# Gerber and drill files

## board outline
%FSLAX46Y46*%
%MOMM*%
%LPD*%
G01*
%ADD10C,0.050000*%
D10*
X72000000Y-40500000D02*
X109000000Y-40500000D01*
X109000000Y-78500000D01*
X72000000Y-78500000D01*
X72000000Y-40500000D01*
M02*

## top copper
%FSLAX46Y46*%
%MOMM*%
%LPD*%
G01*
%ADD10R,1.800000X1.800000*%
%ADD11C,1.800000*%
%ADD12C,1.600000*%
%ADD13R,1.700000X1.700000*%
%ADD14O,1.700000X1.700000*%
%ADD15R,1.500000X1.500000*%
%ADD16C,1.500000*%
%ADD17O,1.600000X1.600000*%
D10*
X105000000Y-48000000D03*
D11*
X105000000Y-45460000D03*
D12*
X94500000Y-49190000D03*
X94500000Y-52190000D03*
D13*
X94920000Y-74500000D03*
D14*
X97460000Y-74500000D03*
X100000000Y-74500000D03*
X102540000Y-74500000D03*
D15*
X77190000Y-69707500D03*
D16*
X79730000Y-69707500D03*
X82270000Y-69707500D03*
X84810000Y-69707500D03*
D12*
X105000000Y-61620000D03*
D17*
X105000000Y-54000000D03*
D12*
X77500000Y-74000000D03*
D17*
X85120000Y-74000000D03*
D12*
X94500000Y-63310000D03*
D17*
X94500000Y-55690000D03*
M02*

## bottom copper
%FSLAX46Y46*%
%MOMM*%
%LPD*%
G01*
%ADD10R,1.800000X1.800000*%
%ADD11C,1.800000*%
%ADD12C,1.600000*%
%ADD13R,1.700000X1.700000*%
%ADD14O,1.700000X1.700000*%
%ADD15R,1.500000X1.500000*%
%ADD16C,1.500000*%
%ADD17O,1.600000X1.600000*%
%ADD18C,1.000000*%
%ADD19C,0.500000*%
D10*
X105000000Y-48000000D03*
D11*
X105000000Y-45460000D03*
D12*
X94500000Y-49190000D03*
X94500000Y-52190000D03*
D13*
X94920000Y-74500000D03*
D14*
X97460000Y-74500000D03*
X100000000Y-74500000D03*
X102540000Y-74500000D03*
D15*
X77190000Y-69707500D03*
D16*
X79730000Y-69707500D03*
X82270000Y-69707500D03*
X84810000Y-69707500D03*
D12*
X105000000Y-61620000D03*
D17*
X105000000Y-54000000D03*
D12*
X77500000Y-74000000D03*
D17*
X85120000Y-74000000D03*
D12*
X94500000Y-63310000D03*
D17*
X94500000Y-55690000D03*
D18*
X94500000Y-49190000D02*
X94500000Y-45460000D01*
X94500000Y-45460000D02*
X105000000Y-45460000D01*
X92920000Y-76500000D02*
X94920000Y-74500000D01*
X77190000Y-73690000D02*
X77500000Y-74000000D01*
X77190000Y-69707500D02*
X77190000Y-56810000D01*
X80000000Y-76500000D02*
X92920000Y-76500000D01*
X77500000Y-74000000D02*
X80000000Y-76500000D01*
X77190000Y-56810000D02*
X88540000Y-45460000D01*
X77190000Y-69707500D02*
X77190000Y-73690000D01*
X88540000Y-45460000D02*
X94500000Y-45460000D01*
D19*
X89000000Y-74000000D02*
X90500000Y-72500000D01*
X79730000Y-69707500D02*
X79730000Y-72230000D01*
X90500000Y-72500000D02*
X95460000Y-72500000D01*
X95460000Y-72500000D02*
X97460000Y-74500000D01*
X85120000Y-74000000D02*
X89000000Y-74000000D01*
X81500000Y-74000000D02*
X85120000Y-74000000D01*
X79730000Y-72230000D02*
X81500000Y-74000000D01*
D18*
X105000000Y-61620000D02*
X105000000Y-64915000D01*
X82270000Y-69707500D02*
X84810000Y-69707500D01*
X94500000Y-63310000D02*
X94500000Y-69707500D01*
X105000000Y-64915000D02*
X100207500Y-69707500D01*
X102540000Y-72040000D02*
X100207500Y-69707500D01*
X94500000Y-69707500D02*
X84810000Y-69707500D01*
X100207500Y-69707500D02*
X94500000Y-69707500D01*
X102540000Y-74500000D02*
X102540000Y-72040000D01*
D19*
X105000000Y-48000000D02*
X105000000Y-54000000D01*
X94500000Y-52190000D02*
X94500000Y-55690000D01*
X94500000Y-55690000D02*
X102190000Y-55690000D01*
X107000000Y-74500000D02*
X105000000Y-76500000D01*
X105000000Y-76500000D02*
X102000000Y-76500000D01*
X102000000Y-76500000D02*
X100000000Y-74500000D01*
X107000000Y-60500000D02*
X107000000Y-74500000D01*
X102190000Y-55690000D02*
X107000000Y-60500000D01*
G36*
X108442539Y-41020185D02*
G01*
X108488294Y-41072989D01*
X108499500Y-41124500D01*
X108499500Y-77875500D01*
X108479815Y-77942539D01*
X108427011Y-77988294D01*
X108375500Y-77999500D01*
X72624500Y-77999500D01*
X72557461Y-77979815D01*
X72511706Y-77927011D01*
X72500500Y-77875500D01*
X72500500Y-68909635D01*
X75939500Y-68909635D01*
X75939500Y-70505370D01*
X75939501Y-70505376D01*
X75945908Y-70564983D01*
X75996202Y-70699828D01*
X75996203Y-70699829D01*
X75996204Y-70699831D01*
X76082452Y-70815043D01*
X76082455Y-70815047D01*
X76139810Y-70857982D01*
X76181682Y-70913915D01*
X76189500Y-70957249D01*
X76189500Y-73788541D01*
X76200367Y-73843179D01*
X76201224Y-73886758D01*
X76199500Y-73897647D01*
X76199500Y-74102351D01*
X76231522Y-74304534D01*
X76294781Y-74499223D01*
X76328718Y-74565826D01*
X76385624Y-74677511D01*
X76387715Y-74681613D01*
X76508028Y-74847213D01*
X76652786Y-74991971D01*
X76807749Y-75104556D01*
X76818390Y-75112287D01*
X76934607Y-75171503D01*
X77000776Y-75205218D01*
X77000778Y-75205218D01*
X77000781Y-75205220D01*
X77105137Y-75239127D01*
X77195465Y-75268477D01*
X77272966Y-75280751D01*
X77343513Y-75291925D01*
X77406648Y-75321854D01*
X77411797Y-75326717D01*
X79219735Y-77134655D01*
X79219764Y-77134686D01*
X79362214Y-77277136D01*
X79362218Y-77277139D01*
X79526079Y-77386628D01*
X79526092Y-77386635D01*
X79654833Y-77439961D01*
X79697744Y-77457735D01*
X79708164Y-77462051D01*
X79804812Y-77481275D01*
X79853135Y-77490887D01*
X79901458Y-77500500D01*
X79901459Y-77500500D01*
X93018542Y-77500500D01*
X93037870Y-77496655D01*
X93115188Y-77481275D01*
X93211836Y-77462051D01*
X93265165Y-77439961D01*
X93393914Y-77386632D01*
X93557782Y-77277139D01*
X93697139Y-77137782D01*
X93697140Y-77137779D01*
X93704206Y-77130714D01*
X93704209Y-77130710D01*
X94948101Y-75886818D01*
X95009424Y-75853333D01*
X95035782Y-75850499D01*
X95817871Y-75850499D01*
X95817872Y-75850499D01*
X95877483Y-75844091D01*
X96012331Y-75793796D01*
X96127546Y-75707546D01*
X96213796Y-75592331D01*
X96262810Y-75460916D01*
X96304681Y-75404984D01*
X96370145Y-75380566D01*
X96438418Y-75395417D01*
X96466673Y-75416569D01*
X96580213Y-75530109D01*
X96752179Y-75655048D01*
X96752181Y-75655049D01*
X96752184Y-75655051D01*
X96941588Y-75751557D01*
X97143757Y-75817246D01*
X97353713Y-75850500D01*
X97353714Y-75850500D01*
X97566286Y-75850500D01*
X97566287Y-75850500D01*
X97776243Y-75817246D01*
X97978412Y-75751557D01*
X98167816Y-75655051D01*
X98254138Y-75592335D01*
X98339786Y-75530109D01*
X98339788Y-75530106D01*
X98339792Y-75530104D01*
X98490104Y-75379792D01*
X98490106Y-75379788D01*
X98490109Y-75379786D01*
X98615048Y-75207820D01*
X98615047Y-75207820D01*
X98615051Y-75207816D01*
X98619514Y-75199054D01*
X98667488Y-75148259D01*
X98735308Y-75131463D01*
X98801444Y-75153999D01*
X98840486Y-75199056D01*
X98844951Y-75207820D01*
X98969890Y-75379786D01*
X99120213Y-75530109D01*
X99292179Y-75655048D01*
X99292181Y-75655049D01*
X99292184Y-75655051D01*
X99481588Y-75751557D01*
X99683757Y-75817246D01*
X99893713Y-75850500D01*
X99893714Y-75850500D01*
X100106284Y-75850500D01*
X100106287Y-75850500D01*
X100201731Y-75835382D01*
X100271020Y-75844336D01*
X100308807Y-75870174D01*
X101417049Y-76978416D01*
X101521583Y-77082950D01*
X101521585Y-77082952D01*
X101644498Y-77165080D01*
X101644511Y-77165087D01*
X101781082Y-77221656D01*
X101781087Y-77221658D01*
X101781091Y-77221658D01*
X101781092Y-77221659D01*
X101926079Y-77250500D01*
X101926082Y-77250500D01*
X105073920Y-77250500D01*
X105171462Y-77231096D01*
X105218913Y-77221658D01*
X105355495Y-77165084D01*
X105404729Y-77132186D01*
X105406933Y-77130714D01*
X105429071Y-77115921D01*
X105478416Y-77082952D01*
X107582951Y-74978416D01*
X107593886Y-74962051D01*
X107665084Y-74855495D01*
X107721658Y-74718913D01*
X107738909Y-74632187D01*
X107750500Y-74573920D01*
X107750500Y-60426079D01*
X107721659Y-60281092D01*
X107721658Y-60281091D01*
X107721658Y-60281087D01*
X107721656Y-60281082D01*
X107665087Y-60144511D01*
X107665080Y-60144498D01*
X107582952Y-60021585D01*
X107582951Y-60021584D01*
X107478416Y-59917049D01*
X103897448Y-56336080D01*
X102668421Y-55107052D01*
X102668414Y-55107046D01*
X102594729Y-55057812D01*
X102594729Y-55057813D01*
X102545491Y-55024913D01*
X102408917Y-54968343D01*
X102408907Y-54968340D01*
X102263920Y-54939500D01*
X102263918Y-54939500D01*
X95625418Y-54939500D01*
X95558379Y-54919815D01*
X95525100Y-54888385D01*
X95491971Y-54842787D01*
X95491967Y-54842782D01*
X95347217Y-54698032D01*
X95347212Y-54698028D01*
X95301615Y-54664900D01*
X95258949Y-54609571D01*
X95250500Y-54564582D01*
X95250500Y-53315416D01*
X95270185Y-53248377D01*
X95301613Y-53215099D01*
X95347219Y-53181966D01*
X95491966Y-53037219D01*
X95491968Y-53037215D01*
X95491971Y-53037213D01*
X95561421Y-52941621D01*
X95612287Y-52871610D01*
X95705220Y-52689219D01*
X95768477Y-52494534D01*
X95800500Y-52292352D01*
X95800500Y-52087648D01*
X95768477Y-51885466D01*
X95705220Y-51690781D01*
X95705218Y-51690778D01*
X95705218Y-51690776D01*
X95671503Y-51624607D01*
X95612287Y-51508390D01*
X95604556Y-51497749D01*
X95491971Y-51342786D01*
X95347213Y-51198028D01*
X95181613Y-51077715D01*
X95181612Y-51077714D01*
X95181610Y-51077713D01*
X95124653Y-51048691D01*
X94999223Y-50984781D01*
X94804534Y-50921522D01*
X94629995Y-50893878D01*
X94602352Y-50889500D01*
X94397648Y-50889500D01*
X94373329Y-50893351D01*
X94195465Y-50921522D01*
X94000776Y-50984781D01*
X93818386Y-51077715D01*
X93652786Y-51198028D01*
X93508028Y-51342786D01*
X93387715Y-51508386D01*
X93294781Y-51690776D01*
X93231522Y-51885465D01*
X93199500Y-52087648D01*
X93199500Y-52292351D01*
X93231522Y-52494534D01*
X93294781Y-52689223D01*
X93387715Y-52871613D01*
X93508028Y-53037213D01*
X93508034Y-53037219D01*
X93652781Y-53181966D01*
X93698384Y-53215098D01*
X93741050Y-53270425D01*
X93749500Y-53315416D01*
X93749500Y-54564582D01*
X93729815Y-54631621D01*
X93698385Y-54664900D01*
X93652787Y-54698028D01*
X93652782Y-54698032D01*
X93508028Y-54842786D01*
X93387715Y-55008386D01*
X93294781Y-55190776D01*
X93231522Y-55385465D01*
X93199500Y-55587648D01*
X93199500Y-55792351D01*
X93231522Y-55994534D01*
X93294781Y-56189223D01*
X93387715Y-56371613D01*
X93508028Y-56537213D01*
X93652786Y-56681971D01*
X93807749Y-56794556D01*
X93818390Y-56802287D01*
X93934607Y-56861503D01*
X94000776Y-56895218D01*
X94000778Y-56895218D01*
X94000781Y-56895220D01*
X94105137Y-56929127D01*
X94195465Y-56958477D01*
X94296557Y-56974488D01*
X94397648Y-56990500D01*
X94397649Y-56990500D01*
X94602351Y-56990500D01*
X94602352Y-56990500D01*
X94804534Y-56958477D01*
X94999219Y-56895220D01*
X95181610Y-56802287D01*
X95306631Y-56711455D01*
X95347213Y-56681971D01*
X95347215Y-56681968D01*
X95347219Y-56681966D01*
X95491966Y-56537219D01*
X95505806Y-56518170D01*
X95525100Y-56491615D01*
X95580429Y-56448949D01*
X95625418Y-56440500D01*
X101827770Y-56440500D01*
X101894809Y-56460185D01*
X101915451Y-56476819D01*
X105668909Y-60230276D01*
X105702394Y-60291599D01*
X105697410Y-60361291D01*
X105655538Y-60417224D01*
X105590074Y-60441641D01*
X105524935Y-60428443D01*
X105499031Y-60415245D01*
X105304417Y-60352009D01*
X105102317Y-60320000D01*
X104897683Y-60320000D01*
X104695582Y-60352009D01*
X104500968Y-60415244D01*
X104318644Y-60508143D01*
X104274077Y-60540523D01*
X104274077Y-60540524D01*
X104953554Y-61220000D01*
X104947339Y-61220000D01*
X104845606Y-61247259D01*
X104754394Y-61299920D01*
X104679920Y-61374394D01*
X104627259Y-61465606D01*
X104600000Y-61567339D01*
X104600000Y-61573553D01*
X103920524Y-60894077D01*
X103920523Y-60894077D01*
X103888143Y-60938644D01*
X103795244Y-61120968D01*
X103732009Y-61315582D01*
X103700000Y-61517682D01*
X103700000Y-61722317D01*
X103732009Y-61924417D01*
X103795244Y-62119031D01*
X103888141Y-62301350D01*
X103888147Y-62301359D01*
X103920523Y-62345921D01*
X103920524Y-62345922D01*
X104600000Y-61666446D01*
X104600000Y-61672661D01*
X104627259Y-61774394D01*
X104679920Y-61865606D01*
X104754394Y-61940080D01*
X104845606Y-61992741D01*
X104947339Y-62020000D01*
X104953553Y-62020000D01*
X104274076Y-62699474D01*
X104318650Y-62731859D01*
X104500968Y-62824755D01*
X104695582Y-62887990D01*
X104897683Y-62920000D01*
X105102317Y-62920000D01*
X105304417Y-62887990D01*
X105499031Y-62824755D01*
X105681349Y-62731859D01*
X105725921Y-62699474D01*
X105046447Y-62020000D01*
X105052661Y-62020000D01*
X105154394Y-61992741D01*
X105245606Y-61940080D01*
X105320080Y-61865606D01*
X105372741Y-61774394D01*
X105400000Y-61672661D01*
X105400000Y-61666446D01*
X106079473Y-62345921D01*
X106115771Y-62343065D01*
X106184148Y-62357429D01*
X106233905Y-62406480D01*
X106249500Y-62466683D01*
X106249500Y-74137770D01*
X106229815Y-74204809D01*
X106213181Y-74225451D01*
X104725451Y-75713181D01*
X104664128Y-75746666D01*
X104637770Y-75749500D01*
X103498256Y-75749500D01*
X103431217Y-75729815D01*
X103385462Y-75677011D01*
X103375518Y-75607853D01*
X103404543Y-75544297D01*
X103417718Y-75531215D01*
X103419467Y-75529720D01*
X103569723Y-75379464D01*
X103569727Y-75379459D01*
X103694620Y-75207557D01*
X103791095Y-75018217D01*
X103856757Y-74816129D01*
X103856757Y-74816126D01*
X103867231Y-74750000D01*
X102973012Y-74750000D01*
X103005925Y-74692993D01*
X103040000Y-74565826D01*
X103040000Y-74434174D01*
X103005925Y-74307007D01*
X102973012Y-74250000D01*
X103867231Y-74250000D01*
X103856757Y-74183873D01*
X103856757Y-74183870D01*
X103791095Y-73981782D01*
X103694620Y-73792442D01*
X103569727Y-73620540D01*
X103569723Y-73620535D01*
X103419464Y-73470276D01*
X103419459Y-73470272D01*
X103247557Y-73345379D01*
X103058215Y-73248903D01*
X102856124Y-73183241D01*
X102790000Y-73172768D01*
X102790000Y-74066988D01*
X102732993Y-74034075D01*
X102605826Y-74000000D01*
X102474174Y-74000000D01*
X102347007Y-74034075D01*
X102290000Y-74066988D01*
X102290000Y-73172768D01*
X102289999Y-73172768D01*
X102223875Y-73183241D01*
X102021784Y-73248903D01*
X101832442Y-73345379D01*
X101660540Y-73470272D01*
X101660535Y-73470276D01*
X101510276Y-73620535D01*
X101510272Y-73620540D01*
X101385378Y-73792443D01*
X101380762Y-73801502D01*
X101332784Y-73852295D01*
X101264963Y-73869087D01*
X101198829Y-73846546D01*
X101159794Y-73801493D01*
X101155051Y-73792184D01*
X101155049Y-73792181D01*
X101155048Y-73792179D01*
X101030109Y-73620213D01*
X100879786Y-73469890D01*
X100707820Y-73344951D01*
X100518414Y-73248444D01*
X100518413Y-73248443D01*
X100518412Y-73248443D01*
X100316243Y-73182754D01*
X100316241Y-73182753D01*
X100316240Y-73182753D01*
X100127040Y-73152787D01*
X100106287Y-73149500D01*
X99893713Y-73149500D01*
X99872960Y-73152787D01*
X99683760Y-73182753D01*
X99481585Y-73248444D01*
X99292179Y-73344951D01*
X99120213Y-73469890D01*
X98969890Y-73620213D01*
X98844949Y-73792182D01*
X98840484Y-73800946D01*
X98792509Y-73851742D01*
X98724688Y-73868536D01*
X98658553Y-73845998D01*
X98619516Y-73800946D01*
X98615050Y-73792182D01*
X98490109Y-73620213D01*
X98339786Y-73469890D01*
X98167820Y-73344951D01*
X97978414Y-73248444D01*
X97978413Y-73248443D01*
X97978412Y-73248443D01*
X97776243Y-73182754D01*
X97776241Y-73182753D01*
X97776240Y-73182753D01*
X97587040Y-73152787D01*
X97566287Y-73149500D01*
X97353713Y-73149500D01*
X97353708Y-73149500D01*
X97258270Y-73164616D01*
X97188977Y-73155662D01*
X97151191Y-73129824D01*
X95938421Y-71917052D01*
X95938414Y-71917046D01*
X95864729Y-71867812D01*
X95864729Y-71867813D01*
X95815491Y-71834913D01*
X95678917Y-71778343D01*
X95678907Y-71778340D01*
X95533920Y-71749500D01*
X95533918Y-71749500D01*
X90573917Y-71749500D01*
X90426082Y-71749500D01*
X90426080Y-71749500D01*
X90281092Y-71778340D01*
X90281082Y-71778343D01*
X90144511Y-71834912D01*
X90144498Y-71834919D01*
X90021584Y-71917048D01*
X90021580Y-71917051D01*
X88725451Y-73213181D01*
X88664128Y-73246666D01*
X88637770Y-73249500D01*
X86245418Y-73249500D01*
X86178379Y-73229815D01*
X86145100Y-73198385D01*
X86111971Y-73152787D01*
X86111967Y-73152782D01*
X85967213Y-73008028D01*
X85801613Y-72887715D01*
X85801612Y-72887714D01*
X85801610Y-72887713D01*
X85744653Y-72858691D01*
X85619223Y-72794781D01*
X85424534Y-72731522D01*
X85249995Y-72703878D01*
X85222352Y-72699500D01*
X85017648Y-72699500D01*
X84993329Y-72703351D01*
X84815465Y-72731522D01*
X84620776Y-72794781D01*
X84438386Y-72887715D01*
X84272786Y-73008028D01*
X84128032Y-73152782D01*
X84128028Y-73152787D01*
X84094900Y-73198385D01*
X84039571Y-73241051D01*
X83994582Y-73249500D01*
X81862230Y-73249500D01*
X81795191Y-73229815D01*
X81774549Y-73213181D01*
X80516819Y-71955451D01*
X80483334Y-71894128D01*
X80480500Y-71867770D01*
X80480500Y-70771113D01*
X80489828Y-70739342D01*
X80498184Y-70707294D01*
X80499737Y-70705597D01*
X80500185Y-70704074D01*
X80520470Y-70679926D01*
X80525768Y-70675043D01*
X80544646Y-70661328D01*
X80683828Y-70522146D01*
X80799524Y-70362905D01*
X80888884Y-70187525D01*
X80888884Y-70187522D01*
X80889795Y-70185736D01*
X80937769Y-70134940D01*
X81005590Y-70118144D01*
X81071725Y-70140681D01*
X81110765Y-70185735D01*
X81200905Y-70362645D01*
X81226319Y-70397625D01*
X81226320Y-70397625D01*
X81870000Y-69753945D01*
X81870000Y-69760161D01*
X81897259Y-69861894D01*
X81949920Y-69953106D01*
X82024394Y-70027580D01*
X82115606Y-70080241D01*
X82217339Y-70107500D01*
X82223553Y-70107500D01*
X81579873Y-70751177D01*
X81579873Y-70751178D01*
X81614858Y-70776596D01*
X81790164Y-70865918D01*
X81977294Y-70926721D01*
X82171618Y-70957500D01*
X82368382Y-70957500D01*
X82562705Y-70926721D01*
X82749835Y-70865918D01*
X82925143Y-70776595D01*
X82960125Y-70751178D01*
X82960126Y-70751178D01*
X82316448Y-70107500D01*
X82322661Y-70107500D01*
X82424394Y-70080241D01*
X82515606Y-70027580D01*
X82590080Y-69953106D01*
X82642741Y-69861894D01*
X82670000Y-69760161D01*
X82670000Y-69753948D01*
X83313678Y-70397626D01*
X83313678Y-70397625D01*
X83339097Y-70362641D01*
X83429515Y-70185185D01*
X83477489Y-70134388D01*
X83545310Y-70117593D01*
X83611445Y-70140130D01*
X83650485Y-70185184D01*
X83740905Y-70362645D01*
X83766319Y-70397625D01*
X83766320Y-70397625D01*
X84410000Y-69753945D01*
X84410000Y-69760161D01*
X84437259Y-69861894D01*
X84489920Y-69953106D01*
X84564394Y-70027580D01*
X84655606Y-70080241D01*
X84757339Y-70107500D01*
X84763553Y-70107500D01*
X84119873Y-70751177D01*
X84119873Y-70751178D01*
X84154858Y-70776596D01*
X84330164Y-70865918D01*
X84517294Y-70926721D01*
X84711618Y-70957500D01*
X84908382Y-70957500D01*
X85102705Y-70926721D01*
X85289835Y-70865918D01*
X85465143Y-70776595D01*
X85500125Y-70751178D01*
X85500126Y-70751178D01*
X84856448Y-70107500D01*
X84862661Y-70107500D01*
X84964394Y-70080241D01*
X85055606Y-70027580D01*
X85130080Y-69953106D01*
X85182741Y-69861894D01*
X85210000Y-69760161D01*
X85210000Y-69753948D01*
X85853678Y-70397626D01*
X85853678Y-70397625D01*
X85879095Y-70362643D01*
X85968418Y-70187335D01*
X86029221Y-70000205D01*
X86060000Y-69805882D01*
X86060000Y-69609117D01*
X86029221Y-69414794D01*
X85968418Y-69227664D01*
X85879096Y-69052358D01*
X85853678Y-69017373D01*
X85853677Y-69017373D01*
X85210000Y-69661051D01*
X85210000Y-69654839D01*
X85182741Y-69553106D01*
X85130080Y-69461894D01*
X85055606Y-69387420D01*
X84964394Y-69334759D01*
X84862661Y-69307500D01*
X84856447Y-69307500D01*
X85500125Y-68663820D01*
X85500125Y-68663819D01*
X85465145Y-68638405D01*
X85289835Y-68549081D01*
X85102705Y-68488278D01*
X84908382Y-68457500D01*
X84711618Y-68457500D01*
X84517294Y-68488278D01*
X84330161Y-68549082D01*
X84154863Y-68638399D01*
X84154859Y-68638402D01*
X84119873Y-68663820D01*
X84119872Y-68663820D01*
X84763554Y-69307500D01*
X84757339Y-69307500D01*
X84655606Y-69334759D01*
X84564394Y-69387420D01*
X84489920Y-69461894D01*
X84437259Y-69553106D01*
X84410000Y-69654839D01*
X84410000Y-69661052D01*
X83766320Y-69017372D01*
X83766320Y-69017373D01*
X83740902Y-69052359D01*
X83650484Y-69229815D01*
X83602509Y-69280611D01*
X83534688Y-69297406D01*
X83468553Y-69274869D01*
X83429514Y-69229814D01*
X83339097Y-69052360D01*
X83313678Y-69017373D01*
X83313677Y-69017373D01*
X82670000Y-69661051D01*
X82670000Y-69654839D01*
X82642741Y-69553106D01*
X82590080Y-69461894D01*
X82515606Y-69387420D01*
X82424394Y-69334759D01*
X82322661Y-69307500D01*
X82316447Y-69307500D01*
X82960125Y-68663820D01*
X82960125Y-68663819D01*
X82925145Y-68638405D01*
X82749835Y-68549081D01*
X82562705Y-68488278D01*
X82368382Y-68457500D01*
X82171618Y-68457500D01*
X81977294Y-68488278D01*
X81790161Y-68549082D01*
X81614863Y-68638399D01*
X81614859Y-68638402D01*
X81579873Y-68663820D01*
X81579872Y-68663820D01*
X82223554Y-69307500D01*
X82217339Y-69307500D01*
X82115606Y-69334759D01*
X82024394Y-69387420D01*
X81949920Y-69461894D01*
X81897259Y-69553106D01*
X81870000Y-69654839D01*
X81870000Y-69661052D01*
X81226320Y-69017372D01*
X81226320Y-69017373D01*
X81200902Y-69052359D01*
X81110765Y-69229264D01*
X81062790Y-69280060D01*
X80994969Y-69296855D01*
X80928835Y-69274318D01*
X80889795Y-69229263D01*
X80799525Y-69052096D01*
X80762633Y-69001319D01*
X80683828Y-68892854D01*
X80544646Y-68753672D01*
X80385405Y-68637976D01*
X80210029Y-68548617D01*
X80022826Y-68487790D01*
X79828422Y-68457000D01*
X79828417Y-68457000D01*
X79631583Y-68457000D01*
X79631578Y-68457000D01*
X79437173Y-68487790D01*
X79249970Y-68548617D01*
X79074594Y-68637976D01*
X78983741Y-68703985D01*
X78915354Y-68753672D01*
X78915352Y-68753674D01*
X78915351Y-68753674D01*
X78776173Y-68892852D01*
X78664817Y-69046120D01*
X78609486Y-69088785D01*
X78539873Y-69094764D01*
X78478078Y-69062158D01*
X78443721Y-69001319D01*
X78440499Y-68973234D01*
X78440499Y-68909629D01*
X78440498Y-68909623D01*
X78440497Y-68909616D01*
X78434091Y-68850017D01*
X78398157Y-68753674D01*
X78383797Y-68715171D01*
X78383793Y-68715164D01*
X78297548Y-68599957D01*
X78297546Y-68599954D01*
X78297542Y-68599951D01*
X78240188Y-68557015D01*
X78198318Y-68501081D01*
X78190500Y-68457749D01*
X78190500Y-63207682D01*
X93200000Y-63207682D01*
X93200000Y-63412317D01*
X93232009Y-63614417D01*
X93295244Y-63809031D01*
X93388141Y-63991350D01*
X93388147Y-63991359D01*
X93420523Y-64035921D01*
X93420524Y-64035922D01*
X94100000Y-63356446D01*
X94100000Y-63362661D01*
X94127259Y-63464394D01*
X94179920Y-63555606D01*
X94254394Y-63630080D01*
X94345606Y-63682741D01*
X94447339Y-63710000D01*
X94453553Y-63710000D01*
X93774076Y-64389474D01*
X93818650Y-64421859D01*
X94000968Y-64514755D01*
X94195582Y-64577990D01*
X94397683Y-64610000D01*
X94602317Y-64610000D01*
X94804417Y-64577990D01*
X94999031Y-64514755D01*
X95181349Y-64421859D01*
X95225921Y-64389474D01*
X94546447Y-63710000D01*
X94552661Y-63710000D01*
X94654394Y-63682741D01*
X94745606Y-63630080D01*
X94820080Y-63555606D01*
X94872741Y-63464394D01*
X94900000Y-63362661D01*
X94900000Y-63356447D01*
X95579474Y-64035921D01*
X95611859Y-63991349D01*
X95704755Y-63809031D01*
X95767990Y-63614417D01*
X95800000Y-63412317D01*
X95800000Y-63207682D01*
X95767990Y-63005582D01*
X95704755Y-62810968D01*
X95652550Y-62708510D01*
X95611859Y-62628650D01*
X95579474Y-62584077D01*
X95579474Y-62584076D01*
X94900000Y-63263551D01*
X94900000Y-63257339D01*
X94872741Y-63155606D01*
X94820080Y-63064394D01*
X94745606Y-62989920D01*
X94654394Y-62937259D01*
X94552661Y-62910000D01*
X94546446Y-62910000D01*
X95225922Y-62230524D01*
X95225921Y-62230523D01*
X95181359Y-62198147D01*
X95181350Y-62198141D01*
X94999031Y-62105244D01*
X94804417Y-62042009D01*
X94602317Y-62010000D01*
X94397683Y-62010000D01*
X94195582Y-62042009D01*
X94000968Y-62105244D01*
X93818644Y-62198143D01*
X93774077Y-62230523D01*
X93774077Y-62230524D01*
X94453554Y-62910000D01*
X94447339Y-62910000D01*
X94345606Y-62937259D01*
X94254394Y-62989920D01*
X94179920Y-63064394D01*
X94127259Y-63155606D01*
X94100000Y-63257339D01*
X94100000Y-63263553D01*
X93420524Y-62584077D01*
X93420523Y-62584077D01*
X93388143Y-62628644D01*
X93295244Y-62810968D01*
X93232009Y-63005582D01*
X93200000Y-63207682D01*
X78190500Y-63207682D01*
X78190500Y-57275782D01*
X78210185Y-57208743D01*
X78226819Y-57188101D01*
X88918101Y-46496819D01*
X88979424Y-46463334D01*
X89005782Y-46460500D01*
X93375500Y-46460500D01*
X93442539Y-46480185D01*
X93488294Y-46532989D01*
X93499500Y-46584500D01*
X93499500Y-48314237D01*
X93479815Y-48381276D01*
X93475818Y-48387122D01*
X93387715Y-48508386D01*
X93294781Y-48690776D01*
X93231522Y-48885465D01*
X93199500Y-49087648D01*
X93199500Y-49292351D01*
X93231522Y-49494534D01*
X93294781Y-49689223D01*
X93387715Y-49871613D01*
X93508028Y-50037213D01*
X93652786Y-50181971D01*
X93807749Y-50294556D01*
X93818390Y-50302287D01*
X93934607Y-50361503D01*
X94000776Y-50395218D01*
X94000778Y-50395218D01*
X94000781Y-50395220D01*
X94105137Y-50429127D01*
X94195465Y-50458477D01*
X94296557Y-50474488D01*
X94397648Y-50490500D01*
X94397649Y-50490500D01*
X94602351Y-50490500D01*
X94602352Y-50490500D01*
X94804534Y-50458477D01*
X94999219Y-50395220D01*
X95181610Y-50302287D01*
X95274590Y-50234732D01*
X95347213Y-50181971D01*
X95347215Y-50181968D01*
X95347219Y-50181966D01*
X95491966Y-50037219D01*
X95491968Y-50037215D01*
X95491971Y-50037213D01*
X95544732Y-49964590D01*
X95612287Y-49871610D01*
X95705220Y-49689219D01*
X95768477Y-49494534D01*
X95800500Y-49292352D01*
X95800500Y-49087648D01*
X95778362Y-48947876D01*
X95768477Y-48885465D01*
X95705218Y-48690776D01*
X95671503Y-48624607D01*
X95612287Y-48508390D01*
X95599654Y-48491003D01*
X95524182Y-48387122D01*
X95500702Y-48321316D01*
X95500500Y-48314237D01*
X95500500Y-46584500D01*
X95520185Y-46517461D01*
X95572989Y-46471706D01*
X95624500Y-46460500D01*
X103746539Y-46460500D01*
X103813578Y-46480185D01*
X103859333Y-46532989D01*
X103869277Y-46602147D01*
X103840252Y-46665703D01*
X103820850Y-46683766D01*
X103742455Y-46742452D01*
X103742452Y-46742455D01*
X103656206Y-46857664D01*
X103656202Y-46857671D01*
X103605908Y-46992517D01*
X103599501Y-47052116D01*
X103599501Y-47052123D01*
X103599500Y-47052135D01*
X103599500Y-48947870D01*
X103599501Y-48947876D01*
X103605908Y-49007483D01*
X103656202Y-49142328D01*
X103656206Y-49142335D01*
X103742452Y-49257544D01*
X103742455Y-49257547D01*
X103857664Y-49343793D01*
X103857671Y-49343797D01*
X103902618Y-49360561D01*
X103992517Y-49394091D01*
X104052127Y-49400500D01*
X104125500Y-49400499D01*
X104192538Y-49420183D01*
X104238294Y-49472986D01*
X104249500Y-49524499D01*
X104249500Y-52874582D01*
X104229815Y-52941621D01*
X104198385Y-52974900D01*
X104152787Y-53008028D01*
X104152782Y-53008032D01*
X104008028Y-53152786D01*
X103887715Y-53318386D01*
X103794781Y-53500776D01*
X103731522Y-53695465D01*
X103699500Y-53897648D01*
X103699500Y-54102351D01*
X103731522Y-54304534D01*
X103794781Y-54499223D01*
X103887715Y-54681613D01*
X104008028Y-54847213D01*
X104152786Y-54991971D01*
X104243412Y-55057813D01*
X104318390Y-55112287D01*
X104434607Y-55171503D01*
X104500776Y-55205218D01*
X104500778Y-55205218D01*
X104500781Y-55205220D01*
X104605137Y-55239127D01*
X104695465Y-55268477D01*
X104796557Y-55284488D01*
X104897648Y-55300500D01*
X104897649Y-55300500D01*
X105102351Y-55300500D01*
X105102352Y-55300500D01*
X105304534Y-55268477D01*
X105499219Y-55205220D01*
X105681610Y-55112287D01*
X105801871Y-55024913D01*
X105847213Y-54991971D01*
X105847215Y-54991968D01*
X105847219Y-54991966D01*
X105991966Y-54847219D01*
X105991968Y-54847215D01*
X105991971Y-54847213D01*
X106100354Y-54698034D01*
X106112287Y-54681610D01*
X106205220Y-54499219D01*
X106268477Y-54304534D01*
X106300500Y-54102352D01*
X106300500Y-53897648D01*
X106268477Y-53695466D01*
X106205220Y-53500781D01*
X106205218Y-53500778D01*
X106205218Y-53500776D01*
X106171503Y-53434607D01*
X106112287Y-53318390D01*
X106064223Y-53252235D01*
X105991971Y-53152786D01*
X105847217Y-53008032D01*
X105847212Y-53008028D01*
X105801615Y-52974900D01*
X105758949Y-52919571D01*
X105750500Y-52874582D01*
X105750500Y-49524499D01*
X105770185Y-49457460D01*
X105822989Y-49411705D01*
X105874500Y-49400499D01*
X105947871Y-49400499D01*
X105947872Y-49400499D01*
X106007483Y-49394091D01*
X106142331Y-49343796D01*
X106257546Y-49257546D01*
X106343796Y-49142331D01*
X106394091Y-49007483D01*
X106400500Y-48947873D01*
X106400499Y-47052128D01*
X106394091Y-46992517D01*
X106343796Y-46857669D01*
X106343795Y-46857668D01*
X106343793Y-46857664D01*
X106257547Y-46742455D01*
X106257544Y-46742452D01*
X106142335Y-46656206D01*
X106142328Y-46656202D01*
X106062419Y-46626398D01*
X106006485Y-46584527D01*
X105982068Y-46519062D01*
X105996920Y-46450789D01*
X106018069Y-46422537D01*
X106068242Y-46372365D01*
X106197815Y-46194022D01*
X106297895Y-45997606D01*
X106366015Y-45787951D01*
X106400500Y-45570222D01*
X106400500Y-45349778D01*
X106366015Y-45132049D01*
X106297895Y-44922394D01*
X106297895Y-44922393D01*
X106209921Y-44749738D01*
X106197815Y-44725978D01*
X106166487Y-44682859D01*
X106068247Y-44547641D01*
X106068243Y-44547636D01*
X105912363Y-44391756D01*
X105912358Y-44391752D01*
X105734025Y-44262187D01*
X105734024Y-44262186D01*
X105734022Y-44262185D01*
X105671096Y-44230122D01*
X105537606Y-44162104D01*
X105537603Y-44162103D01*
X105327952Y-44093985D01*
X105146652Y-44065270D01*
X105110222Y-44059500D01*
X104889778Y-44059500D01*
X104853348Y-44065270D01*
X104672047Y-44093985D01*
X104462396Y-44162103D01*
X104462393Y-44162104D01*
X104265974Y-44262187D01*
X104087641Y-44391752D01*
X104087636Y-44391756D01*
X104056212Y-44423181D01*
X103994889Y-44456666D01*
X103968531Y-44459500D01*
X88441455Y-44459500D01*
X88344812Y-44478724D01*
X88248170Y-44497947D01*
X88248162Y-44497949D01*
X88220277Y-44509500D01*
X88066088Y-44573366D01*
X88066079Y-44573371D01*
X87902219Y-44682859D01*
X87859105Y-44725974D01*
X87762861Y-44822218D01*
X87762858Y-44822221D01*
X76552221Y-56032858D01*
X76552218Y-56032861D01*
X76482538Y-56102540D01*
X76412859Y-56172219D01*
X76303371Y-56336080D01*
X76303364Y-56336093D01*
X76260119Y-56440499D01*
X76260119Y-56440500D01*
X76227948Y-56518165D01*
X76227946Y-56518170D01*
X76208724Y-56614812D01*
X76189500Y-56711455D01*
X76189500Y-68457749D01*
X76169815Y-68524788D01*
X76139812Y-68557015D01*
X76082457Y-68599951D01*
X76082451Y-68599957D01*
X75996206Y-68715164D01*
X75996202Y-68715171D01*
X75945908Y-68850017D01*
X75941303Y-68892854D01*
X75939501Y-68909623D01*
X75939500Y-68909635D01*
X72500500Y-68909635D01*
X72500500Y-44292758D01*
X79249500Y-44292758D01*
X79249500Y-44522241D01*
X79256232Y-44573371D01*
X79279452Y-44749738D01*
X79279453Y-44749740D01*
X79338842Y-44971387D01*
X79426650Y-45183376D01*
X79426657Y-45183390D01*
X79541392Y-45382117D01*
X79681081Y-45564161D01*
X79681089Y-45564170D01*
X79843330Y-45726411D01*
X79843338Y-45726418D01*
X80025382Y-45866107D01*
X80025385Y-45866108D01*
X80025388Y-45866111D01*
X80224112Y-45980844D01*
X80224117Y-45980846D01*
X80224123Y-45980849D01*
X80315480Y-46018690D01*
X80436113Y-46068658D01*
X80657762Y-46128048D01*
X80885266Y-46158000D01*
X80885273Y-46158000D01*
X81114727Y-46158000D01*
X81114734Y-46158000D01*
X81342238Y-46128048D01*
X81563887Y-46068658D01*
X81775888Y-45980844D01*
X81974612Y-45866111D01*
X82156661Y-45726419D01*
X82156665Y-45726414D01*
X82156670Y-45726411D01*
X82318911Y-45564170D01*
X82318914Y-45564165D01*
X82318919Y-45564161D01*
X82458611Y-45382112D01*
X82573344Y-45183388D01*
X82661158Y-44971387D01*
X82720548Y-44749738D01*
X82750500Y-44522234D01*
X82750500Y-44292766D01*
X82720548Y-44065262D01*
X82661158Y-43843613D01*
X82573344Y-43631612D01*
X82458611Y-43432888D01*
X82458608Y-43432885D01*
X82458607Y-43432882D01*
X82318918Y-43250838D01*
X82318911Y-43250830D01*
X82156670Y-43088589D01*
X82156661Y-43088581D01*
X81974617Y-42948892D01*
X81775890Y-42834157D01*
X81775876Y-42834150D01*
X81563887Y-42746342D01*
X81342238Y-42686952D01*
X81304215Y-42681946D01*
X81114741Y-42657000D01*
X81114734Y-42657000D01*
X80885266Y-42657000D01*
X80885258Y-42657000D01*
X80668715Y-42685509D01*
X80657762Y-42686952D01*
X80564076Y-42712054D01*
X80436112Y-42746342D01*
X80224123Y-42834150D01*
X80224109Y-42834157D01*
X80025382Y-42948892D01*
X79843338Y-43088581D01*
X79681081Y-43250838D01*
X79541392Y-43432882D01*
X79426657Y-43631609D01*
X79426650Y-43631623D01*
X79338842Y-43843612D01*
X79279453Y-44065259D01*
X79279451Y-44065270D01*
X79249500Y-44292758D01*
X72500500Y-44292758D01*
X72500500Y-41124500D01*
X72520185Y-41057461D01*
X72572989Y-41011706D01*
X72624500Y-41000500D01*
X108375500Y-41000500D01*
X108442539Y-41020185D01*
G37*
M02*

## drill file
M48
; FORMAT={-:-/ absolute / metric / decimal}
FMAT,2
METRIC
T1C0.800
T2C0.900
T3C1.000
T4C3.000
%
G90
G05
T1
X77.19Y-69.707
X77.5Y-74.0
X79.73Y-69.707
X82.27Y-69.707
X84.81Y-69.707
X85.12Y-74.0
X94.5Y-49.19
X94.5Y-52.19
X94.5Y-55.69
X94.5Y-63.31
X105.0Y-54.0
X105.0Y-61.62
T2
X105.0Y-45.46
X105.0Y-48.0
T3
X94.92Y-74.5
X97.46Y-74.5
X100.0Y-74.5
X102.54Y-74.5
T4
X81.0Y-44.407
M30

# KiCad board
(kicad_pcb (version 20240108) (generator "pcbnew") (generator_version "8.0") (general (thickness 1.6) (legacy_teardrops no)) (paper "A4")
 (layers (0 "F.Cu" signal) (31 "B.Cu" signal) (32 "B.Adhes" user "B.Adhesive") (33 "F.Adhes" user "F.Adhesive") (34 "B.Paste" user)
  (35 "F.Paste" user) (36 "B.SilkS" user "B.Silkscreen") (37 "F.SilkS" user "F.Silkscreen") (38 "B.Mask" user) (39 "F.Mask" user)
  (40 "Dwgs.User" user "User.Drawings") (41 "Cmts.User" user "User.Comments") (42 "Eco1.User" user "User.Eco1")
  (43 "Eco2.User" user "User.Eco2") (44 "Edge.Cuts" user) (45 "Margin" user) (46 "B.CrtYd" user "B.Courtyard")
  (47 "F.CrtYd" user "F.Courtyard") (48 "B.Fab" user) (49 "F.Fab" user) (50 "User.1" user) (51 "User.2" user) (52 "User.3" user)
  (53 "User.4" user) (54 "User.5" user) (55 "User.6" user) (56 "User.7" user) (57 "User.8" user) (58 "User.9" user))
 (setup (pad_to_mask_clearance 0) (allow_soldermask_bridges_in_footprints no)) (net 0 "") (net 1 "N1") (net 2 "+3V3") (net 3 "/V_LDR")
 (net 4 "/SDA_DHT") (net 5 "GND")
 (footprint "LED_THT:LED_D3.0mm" (layer "F.Cu") (at 105 48 90)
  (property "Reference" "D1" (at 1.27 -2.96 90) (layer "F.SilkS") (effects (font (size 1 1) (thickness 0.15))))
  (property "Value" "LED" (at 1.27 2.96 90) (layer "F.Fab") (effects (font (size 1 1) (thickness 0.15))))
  (pad "1" thru_hole rect (at 0 0 90) (size 1.8 1.8) (drill 0.9) (layers "*.Cu" "*.Mask") (remove_unused_layers no) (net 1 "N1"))
  (pad "2" thru_hole circle (at 2.54 0 90) (size 1.8 1.8) (drill 0.9) (layers "*.Cu" "*.Mask") (remove_unused_layers no) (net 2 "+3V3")))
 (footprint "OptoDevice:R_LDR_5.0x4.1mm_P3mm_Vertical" (layer "F.Cu") (at 94.5 49.19 -90)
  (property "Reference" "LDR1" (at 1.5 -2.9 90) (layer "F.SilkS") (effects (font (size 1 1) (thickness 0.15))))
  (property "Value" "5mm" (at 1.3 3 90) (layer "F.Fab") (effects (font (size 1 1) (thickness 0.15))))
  (pad "1" thru_hole circle (at 0 0 270) (size 1.6 1.6) (drill 0.8) (layers "*.Cu" "*.Mask") (remove_unused_layers no) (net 2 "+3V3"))
  (pad "2" thru_hole circle (at 3 0 270) (size 1.6 1.6) (drill 0.8) (layers "*.Cu" "*.Mask") (remove_unused_layers no) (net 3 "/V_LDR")))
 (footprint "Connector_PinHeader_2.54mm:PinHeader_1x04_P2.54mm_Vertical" (layer "F.Cu") (at 94.92 74.5 90)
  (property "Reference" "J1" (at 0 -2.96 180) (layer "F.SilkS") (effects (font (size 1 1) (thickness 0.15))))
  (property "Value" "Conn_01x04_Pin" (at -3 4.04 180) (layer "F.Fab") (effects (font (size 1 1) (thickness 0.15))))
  (pad "1" thru_hole rect (at 0 0 90) (size 1.7 1.7) (drill 1) (layers "*.Cu" "*.Mask") (remove_unused_layers no) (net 2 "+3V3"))
  (pad "2" thru_hole oval (at 0 2.54 90) (size 1.7 1.7) (drill 1) (layers "*.Cu" "*.Mask") (remove_unused_layers no) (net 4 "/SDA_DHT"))
  (pad "3" thru_hole oval (at 0 5.08 90) (size 1.7 1.7) (drill 1) (layers "*.Cu" "*.Mask") (remove_unused_layers no) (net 3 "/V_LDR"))
  (pad "4" thru_hole oval (at 0 7.62 90) (size 1.7 1.7) (drill 1) (layers "*.Cu" "*.Mask") (remove_unused_layers no) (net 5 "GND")))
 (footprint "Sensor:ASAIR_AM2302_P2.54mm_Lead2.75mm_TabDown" (layer "F.Cu") (at 77.19 69.7075 90)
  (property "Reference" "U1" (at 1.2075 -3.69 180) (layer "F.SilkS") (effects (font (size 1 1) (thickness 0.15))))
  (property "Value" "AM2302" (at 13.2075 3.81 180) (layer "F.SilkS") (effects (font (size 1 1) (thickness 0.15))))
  (pad "" np_thru_hole circle (at 25.3 3.81 90) (size 3 3) (drill 3) (layers "F&B.Cu" "*.Mask"))
  (pad "1" thru_hole rect (at 0 0 90) (size 1.5 1.5) (drill 0.8) (layers "*.Cu" "*.Mask") (remove_unused_layers no) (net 2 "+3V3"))
  (pad "2" thru_hole circle (at 0 2.54 90) (size 1.5 1.5) (drill 0.8) (layers "*.Cu" "*.Mask") (remove_unused_layers no) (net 4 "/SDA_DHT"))
  (pad "3" thru_hole circle (at 0 5.08 90) (size 1.5 1.5) (drill 0.8) (layers "*.Cu" "*.Mask") (remove_unused_layers no) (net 5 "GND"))
  (pad "4" thru_hole circle (at 0 7.62 90) (size 1.5 1.5) (drill 0.8) (layers "*.Cu" "*.Mask") (remove_unused_layers no) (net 5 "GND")))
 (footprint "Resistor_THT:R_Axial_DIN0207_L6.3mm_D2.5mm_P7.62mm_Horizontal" (layer "F.Cu") (at 105 61.62 90)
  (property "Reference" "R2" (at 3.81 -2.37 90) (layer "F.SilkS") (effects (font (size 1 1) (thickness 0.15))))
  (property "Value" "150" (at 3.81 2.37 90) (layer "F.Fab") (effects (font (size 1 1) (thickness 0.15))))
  (pad "1" thru_hole circle (at 0 0 90) (size 1.6 1.6) (drill 0.8) (layers "*.Cu" "*.Mask") (remove_unused_layers no) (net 5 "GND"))
  (pad "2" thru_hole oval (at 7.62 0 90) (size 1.6 1.6) (drill 0.8) (layers "*.Cu" "*.Mask") (remove_unused_layers no) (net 1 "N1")))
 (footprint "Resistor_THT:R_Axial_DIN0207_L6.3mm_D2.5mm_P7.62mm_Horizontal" (layer "F.Cu") (at 77.5 74)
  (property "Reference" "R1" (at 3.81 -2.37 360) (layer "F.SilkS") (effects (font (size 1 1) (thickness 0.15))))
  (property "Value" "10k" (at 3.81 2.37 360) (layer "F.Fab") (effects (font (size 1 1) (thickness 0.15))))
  (pad "1" thru_hole circle (at 0 0) (size 1.6 1.6) (drill 0.8) (layers "*.Cu" "*.Mask") (remove_unused_layers no) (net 2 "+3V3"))
  (pad "2" thru_hole oval (at 7.62 0) (size 1.6 1.6) (drill 0.8) (layers "*.Cu" "*.Mask") (remove_unused_layers no) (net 4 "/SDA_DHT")))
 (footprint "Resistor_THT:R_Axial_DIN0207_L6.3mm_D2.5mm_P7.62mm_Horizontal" (layer "F.Cu") (at 94.5 63.31 90)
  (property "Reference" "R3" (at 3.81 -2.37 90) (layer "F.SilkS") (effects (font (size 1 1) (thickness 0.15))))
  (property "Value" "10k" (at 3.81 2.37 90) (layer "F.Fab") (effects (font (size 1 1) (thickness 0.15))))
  (pad "1" thru_hole circle (at 0 0 90) (size 1.6 1.6) (drill 0.8) (layers "*.Cu" "*.Mask") (remove_unused_layers no) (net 5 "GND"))
  (pad "2" thru_hole oval (at 7.62 0 90) (size 1.6 1.6) (drill 0.8) (layers "*.Cu" "*.Mask") (remove_unused_layers no) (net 3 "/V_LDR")))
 (gr_rect (start 72 40.5) (end 109 78.5) (stroke (width 0.05) (type default)) (fill none) (layer "Edge.Cuts"))
 (segment (start 94.5 49.19) (end 94.5 45.46) (width 1) (layer "B.Cu") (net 2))
 (segment (start 94.5 45.46) (end 105 45.46) (width 1) (layer "B.Cu") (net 2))
 (segment (start 92.92 76.5) (end 94.92 74.5) (width 1) (layer "B.Cu") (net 2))
 (segment (start 77.19 73.69) (end 77.5 74) (width 1) (layer "B.Cu") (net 2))
 (segment (start 77.19 69.7075) (end 77.19 56.81) (width 1) (layer "B.Cu") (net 2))
 (segment (start 80 76.5) (end 92.92 76.5) (width 1) (layer "B.Cu") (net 2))
 (segment (start 77.5 74) (end 80 76.5) (width 1) (layer "B.Cu") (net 2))
 (segment (start 77.19 56.81) (end 88.54 45.46) (width 1) (layer "B.Cu") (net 2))
 (segment (start 77.19 69.7075) (end 77.19 73.69) (width 1) (layer "B.Cu") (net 2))
 (segment (start 88.54 45.46) (end 94.5 45.46) (width 1) (layer "B.Cu") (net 2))
 (segment (start 89 74) (end 90.5 72.5) (width 0.5) (layer "B.Cu") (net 4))
 (segment (start 79.73 69.7075) (end 79.73 72.23) (width 0.5) (layer "B.Cu") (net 4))
 (segment (start 90.5 72.5) (end 95.46 72.5) (width 0.5) (layer "B.Cu") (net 4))
 (segment (start 95.46 72.5) (end 97.46 74.5) (width 0.5) (layer "B.Cu") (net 4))
 (segment (start 85.12 74) (end 89 74) (width 0.5) (layer "B.Cu") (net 4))
 (segment (start 81.5 74) (end 85.12 74) (width 0.5) (layer "B.Cu") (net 4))
 (segment (start 79.73 72.23) (end 81.5 74) (width 0.5) (layer "B.Cu") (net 4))
 (segment (start 105 61.62) (end 105 64.915) (width 1) (layer "B.Cu") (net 5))
 (segment (start 82.27 69.7075) (end 84.81 69.7075) (width 1) (layer "B.Cu") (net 5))
 (segment (start 94.5 63.31) (end 94.5 69.7075) (width 1) (layer "B.Cu") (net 5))
 (segment (start 105 64.915) (end 100.2075 69.7075) (width 1) (layer "B.Cu") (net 5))
 (segment (start 102.54 72.04) (end 100.2075 69.7075) (width 1) (layer "B.Cu") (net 5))
 (segment (start 94.5 69.7075) (end 84.81 69.7075) (width 1) (layer "B.Cu") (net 5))
 (segment (start 100.2075 69.7075) (end 94.5 69.7075) (width 1) (layer "B.Cu") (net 5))
 (segment (start 102.54 74.5) (end 102.54 72.04) (width 1) (layer "B.Cu") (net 5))
 (segment (start 105 48) (end 105 54) (width 0.5) (layer "B.Cu") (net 1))
 (segment (start 94.5 52.19) (end 94.5 55.69) (width 0.5) (layer "B.Cu") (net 3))
 (segment (start 94.5 55.69) (end 102.19 55.69) (width 0.5) (layer "B.Cu") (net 3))
 (segment (start 107 74.5) (end 105 76.5) (width 0.5) (layer "B.Cu") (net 3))
 (segment (start 105 76.5) (end 102 76.5) (width 0.5) (layer "B.Cu") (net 3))
 (segment (start 102 76.5) (end 100 74.5) (width 0.5) (layer "B.Cu") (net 3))
 (segment (start 107 60.5) (end 107 74.5) (width 0.5) (layer "B.Cu") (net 3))
 (segment (start 102.19 55.69) (end 107 60.5) (width 0.5) (layer "B.Cu") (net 3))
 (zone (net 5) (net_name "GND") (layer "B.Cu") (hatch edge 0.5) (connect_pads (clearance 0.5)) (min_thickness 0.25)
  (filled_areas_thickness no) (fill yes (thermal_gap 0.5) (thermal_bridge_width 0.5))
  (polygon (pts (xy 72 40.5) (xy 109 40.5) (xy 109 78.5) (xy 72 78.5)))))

